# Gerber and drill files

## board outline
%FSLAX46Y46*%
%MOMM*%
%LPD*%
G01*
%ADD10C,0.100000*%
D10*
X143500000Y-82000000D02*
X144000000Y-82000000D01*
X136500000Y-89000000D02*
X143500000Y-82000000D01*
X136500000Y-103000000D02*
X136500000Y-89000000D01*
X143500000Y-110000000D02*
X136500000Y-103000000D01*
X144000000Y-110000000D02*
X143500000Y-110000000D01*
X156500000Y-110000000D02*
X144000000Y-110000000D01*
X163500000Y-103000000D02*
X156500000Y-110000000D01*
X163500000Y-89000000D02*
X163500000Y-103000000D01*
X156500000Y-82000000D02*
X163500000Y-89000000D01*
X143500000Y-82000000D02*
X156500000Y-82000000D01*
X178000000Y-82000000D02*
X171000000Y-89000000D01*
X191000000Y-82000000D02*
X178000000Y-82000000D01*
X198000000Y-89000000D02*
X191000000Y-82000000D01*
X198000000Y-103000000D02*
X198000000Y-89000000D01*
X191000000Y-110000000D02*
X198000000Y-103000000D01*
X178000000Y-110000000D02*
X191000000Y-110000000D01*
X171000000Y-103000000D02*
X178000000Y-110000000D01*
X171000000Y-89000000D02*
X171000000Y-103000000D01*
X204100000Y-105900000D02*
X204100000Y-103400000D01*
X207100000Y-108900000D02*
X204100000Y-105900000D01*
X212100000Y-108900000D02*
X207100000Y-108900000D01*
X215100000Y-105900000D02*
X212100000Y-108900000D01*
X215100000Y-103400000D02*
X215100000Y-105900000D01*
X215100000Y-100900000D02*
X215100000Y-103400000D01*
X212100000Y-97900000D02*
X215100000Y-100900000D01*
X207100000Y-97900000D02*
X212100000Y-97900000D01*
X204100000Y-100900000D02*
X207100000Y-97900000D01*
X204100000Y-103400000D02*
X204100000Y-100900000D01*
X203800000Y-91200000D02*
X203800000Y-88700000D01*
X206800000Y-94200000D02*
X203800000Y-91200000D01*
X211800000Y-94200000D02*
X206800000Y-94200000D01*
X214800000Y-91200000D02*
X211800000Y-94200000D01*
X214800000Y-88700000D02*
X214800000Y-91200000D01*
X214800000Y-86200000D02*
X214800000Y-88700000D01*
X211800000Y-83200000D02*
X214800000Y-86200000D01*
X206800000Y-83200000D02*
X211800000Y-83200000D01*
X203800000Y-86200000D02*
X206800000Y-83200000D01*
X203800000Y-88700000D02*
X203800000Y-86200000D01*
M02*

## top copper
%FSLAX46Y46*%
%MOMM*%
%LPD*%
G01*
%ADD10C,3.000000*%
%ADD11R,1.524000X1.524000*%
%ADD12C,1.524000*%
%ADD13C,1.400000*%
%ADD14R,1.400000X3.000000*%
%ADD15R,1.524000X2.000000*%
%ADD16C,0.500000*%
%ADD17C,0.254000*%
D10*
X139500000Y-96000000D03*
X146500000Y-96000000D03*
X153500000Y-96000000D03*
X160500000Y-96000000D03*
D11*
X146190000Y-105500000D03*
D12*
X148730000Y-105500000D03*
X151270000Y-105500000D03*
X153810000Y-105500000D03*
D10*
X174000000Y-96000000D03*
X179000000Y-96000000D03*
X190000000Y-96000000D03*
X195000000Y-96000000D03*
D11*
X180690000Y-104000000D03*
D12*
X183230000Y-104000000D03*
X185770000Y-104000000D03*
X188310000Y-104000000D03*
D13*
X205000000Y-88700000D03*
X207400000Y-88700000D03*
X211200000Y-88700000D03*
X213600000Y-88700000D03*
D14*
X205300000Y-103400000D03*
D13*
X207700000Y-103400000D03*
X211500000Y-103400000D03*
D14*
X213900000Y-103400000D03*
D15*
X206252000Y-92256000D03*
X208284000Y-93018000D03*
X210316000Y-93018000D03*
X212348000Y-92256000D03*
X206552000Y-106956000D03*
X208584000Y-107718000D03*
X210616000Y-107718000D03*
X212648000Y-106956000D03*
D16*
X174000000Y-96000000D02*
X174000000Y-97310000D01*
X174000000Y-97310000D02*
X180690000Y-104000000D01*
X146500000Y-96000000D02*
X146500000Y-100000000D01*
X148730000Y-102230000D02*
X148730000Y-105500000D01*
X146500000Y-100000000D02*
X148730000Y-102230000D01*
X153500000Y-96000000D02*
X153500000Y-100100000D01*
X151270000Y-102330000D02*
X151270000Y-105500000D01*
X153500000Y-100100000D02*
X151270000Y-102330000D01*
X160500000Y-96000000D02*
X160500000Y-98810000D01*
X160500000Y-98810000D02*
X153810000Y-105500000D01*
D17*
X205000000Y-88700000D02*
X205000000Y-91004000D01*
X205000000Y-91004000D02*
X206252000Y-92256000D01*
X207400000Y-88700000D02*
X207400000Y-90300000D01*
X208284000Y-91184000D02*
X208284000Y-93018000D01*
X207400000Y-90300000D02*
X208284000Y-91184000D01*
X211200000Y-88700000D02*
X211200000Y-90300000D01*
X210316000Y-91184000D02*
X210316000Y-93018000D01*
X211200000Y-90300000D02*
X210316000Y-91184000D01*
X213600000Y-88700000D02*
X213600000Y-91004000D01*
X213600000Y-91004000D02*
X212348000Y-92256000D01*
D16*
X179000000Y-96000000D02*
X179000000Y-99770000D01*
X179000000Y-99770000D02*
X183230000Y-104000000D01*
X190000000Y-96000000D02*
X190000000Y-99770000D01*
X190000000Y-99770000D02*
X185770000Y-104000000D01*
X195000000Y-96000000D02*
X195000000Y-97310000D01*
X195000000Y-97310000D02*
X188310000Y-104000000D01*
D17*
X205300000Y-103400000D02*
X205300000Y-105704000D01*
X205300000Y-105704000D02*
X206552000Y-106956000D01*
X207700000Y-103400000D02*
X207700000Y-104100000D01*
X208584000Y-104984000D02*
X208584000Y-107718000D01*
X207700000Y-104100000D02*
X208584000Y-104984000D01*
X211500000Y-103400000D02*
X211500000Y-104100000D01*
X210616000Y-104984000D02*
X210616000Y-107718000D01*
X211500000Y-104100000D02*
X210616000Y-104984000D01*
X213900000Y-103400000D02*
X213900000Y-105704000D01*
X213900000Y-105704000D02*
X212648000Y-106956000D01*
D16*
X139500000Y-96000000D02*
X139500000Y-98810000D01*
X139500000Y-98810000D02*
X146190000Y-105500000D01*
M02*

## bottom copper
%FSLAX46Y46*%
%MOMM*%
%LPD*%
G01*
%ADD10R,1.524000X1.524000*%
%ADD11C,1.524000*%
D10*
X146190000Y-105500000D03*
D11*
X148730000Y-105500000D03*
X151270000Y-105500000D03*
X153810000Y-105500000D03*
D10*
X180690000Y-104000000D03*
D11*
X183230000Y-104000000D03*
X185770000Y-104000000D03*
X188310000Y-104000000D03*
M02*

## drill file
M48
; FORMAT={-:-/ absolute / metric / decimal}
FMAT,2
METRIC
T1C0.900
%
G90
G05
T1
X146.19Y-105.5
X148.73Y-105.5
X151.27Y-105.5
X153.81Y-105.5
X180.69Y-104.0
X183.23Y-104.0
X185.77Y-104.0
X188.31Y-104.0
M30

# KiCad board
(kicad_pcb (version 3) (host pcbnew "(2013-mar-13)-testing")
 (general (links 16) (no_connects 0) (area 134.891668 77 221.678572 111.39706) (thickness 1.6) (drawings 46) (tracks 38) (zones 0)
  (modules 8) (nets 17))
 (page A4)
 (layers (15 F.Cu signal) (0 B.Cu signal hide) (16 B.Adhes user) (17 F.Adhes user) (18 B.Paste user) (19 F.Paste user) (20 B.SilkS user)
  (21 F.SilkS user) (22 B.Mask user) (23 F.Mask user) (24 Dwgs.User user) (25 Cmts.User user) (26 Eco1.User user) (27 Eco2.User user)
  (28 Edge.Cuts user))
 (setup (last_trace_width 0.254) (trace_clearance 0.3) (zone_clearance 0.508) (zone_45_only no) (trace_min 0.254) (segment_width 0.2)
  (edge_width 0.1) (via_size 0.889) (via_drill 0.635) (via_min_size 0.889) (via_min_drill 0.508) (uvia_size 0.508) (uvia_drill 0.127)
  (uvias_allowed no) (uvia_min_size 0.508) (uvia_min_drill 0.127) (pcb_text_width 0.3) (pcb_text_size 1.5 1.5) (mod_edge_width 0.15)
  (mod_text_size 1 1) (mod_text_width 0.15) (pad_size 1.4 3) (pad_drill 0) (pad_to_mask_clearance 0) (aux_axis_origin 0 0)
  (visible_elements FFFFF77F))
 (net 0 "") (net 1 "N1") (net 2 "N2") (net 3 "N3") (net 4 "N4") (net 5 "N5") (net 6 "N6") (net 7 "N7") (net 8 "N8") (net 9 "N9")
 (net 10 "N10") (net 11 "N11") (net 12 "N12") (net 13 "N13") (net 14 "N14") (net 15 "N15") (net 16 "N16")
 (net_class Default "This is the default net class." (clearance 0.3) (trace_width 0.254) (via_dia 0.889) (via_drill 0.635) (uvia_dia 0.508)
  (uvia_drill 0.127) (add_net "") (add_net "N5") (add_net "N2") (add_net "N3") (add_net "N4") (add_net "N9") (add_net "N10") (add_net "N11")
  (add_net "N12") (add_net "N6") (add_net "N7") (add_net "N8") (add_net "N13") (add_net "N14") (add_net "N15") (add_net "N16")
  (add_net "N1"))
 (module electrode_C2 (layer F.Cu) (at 150 96)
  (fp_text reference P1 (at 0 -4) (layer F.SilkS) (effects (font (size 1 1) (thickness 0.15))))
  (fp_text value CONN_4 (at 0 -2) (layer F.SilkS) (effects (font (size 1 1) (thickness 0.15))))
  (pad 1 smd circle (at -10.5 0) (size 3 3) (layers F.Cu F.Paste F.Mask) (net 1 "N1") (solder_mask_margin 0.1))
  (pad 2 smd circle (at -3.5 0) (size 3 3) (layers F.Cu F.Paste F.Mask) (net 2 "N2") (solder_mask_margin 0.1))
  (pad 3 smd circle (at 3.5 0) (size 3 3) (layers F.Cu F.Paste F.Mask) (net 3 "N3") (solder_mask_margin 0.1))
  (pad 4 smd circle (at 10.5 0) (size 3 3) (layers F.Cu F.Paste F.Mask) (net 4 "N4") (solder_mask_margin 0.1)))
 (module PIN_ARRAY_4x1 (layer F.Cu) (at 150 105.5)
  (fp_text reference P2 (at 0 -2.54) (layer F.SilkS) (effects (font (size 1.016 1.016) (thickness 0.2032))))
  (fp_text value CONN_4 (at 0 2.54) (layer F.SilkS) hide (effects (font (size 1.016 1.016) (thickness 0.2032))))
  (pad 1 thru_hole rect (at -3.81 0) (size 1.524 1.524) (drill 0.9) (layers *.Cu *.Mask F.SilkS) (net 1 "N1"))
  (pad 2 thru_hole circle (at -1.27 0) (size 1.524 1.524) (drill 0.9) (layers *.Cu *.Mask F.SilkS) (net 2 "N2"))
  (pad 3 thru_hole circle (at 1.27 0) (size 1.524 1.524) (drill 0.9) (layers *.Cu *.Mask F.SilkS) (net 3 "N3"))
  (pad 4 thru_hole circle (at 3.81 0) (size 1.524 1.524) (drill 0.9) (layers *.Cu *.Mask F.SilkS) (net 4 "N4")))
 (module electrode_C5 (layer F.Cu) (at 184.5 96)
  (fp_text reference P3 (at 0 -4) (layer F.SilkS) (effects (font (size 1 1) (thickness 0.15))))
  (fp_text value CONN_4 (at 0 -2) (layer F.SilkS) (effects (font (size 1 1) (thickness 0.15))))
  (pad 1 smd circle (at -10.5 0) (size 3 3) (layers F.Cu F.Paste F.Mask) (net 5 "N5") (solder_mask_margin 0.1))
  (pad 2 smd circle (at -5.5 0) (size 3 3) (layers F.Cu F.Paste F.Mask) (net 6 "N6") (solder_mask_margin 0.1))
  (pad 3 smd circle (at 5.5 0) (size 3 3) (layers F.Cu F.Paste F.Mask) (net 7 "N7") (solder_mask_margin 0.1))
  (pad 4 smd circle (at 10.5 0) (size 3 3) (layers F.Cu F.Paste F.Mask) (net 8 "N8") (solder_mask_margin 0.1)))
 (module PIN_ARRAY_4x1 (layer F.Cu) (at 184.5 104)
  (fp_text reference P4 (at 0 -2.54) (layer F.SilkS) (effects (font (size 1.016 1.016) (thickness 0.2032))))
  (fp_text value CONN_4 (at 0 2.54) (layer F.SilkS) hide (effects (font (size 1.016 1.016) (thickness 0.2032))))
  (pad 1 thru_hole rect (at -3.81 0) (size 1.524 1.524) (drill 0.9) (layers *.Cu *.Mask F.SilkS) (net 5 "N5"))
  (pad 2 thru_hole circle (at -1.27 0) (size 1.524 1.524) (drill 0.9) (layers *.Cu *.Mask F.SilkS) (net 6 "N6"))
  (pad 3 thru_hole circle (at 1.27 0) (size 1.524 1.524) (drill 0.9) (layers *.Cu *.Mask F.SilkS) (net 7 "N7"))
  (pad 4 thru_hole circle (at 3.81 0) (size 1.524 1.524) (drill 0.9) (layers *.Cu *.Mask F.SilkS) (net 8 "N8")))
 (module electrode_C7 (layer F.Cu) (at 209.3 88.7)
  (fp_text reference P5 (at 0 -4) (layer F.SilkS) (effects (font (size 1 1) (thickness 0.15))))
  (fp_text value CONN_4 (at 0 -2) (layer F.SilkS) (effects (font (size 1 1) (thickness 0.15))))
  (pad 1 smd circle (at -4.3 0) (size 1.4 1.4) (layers F.Cu F.Paste F.Mask) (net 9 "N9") (solder_mask_margin 0.1))
  (pad 2 smd circle (at -1.9 0) (size 1.4 1.4) (layers F.Cu F.Paste F.Mask) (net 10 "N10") (solder_mask_margin 0.1))
  (pad 3 smd circle (at 1.9 0) (size 1.4 1.4) (layers F.Cu F.Paste F.Mask) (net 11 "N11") (solder_mask_margin 0.1))
  (pad 4 smd circle (at 4.3 0) (size 1.4 1.4) (layers F.Cu F.Paste F.Mask) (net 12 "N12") (solder_mask_margin 0.1)))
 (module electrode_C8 (layer F.Cu) (at 209.6 103.4)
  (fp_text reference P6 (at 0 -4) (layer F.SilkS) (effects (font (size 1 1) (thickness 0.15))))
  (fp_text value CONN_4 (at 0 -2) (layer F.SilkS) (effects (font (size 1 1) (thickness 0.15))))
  (pad 1 smd rect (at -4.3 0) (size 1.4 3) (layers F.Cu F.Paste F.Mask) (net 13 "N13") (solder_mask_margin 0.1))
  (pad 2 smd circle (at -1.9 0) (size 1.4 1.4) (layers F.Cu F.Paste F.Mask) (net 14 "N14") (solder_mask_margin 0.1))
  (pad 3 smd circle (at 1.9 0) (size 1.4 1.4) (layers F.Cu F.Paste F.Mask) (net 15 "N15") (solder_mask_margin 0.1))
  (pad 4 smd rect (at 4.3 0) (size 1.4 3) (layers F.Cu F.Paste F.Mask) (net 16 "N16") (solder_mask_margin 0.1)))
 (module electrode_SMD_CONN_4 (layer F.Cu) (at 209.3 88.7)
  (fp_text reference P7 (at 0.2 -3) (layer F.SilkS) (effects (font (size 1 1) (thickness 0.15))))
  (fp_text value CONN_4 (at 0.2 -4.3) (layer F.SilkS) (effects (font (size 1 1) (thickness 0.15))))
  (pad 1 smd rect (at -3.048 3.556) (size 1.524 2) (layers F.Cu F.Paste F.Mask) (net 9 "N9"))
  (pad 2 smd rect (at -1.016 4.318) (size 1.524 2) (layers F.Cu F.Paste F.Mask) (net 10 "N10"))
  (pad 3 smd rect (at 1.016 4.318) (size 1.524 2) (layers F.Cu F.Paste F.Mask) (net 11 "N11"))
  (pad 4 smd rect (at 3.048 3.556) (size 1.524 2) (layers F.Cu F.Paste F.Mask) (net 12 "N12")))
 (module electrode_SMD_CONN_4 (layer F.Cu) (at 209.6 103.4)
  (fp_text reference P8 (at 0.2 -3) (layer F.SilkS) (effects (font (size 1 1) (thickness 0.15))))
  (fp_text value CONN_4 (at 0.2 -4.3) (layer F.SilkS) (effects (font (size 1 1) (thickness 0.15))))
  (pad 1 smd rect (at -3.048 3.556) (size 1.524 2) (layers F.Cu F.Paste F.Mask) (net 13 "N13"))
  (pad 2 smd rect (at -1.016 4.318) (size 1.524 2) (layers F.Cu F.Paste F.Mask) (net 14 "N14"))
  (pad 3 smd rect (at 1.016 4.318) (size 1.524 2) (layers F.Cu F.Paste F.Mask) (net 15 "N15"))
  (pad 4 smd rect (at 3.048 3.556) (size 1.524 2) (layers F.Cu F.Paste F.Mask) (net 16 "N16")))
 (gr_line (start 143.5 82) (end 144 82) (angle 90) (layer Edge.Cuts) (width 0.1))
 (gr_line (start 136.5 89) (end 143.5 82) (angle 90) (layer Edge.Cuts) (width 0.1))
 (gr_line (start 136.5 103) (end 136.5 89) (angle 90) (layer Edge.Cuts) (width 0.1))
 (gr_line (start 143.5 110) (end 136.5 103) (angle 90) (layer Edge.Cuts) (width 0.1))
 (gr_line (start 144 110) (end 143.5 110) (angle 90) (layer Edge.Cuts) (width 0.1))
 (gr_line (start 156.5 110) (end 144 110) (angle 90) (layer Edge.Cuts) (width 0.1))
 (gr_line (start 163.5 103) (end 156.5 110) (angle 90) (layer Edge.Cuts) (width 0.1))
 (gr_line (start 163.5 89) (end 163.5 103) (angle 90) (layer Edge.Cuts) (width 0.1))
 (gr_line (start 156.5 82) (end 163.5 89) (angle 90) (layer Edge.Cuts) (width 0.1))
 (gr_line (start 143.5 82) (end 156.5 82) (angle 90) (layer Edge.Cuts) (width 0.1))
 (gr_line (start 178 82) (end 171 89) (angle 90) (layer Edge.Cuts) (width 0.1))
 (gr_line (start 191 82) (end 178 82) (angle 90) (layer Edge.Cuts) (width 0.1))
 (gr_line (start 198 89) (end 191 82) (angle 90) (layer Edge.Cuts) (width 0.1))
 (gr_line (start 198 103) (end 198 89) (angle 90) (layer Edge.Cuts) (width 0.1))
 (gr_line (start 191 110) (end 198 103) (angle 90) (layer Edge.Cuts) (width 0.1))
 (gr_line (start 178 110) (end 191 110) (angle 90) (layer Edge.Cuts) (width 0.1))
 (gr_line (start 171 103) (end 178 110) (angle 90) (layer Edge.Cuts) (width 0.1))
 (gr_line (start 171 89) (end 171 103) (angle 90) (layer Edge.Cuts) (width 0.1))
 (gr_line (start 204.1 105.9) (end 204.1 103.4) (angle 90) (layer Edge.Cuts) (width 0.1))
 (gr_line (start 207.1 108.9) (end 204.1 105.9) (angle 90) (layer Edge.Cuts) (width 0.1))
 (gr_line (start 212.1 108.9) (end 207.1 108.9) (angle 90) (layer Edge.Cuts) (width 0.1))
 (gr_line (start 215.1 105.9) (end 212.1 108.9) (angle 90) (layer Edge.Cuts) (width 0.1))
 (gr_line (start 215.1 103.4) (end 215.1 105.9) (angle 90) (layer Edge.Cuts) (width 0.1))
 (gr_line (start 215.1 100.9) (end 215.1 103.4) (angle 90) (layer Edge.Cuts) (width 0.1))
 (gr_line (start 212.1 97.9) (end 215.1 100.9) (angle 90) (layer Edge.Cuts) (width 0.1))
 (gr_line (start 207.1 97.9) (end 212.1 97.9) (angle 90) (layer Edge.Cuts) (width 0.1))
 (gr_line (start 204.1 100.9) (end 207.1 97.9) (angle 90) (layer Edge.Cuts) (width 0.1))
 (gr_line (start 204.1 103.4) (end 204.1 100.9) (angle 90) (layer Edge.Cuts) (width 0.1))
 (gr_line (start 203.8 91.2) (end 203.8 88.7) (angle 90) (layer Edge.Cuts) (width 0.1))
 (gr_line (start 206.8 94.2) (end 203.8 91.2) (angle 90) (layer Edge.Cuts) (width 0.1))
 (gr_line (start 211.8 94.2) (end 206.8 94.2) (angle 90) (layer Edge.Cuts) (width 0.1))
 (gr_line (start 214.8 91.2) (end 211.8 94.2) (angle 90) (layer Edge.Cuts) (width 0.1))
 (gr_line (start 214.8 88.7) (end 214.8 91.2) (angle 90) (layer Edge.Cuts) (width 0.1))
 (gr_line (start 214.8 86.2) (end 214.8 88.7) (angle 90) (layer Edge.Cuts) (width 0.1))
 (gr_line (start 211.8 83.2) (end 214.8 86.2) (angle 90) (layer Edge.Cuts) (width 0.1))
 (gr_line (start 206.8 83.2) (end 211.8 83.2) (angle 90) (layer Edge.Cuts) (width 0.1))
 (gr_line (start 203.8 86.2) (end 206.8 83.2) (angle 90) (layer Edge.Cuts) (width 0.1))
 (gr_line (start 203.8 88.7) (end 203.8 86.2) (angle 90) (layer Edge.Cuts) (width 0.1))
 (segment (start 174 96) (end 174 97.31) (width 0.5) (layer F.Cu) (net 5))
 (segment (start 174 97.31) (end 180.69 104) (width 0.5) (layer F.Cu) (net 5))
 (segment (start 146.5 96) (end 146.5 100) (width 0.5) (layer F.Cu) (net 2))
 (segment (start 148.73 102.23) (end 148.73 105.5) (width 0.5) (layer F.Cu) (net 2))
 (segment (start 146.5 100) (end 148.73 102.23) (width 0.5) (layer F.Cu) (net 2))
 (segment (start 153.5 96) (end 153.5 100.1) (width 0.5) (layer F.Cu) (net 3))
 (segment (start 151.27 102.33) (end 151.27 105.5) (width 0.5) (layer F.Cu) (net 3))
 (segment (start 153.5 100.1) (end 151.27 102.33) (width 0.5) (layer F.Cu) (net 3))
 (segment (start 160.5 96) (end 160.5 98.81) (width 0.5) (layer F.Cu) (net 4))
 (segment (start 160.5 98.81) (end 153.81 105.5) (width 0.5) (layer F.Cu) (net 4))
 (segment (start 205 88.7) (end 205 91.004) (width 0.254) (layer F.Cu) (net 9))
 (segment (start 205 91.004) (end 206.252 92.256) (width 0.254) (layer F.Cu) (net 9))
 (segment (start 207.4 88.7) (end 207.4 90.3) (width 0.254) (layer F.Cu) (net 10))
 (segment (start 208.284 91.184) (end 208.284 93.018) (width 0.254) (layer F.Cu) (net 10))
 (segment (start 207.4 90.3) (end 208.284 91.184) (width 0.254) (layer F.Cu) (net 10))
 (segment (start 211.2 88.7) (end 211.2 90.3) (width 0.254) (layer F.Cu) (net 11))
 (segment (start 210.316 91.184) (end 210.316 93.018) (width 0.254) (layer F.Cu) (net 11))
 (segment (start 211.2 90.3) (end 210.316 91.184) (width 0.254) (layer F.Cu) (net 11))
 (segment (start 213.6 88.7) (end 213.6 91.004) (width 0.254) (layer F.Cu) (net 12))
 (segment (start 213.6 91.004) (end 212.348 92.256) (width 0.254) (layer F.Cu) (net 12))
 (segment (start 179 96) (end 179 99.77) (width 0.5) (layer F.Cu) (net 6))
 (segment (start 179 99.77) (end 183.23 104) (width 0.5) (layer F.Cu) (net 6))
 (segment (start 190 96) (end 190 99.77) (width 0.5) (layer F.Cu) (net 7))
 (segment (start 190 99.77) (end 185.77 104) (width 0.5) (layer F.Cu) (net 7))
 (segment (start 195 96) (end 195 97.31) (width 0.5) (layer F.Cu) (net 8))
 (segment (start 195 97.31) (end 188.31 104) (width 0.5) (layer F.Cu) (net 8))
 (segment (start 205.3 103.4) (end 205.3 105.704) (width 0.254) (layer F.Cu) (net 13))
 (segment (start 205.3 105.704) (end 206.552 106.956) (width 0.254) (layer F.Cu) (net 13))
 (segment (start 207.7 103.4) (end 207.7 104.1) (width 0.254) (layer F.Cu) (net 14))
 (segment (start 208.584 104.984) (end 208.584 107.718) (width 0.254) (layer F.Cu) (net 14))
 (segment (start 207.7 104.1) (end 208.584 104.984) (width 0.254) (layer F.Cu) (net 14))
 (segment (start 211.5 103.4) (end 211.5 104.1) (width 0.254) (layer F.Cu) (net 15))
 (segment (start 210.616 104.984) (end 210.616 107.718) (width 0.254) (layer F.Cu) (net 15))
 (segment (start 211.5 104.1) (end 210.616 104.984) (width 0.254) (layer F.Cu) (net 15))
 (segment (start 213.9 103.4) (end 213.9 105.704) (width 0.254) (layer F.Cu) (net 16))
 (segment (start 213.9 105.704) (end 212.648 106.956) (width 0.254) (layer F.Cu) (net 16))
 (segment (start 139.5 96) (end 139.5 98.81) (width 0.5) (layer F.Cu) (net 1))
 (segment (start 139.5 98.81) (end 146.19 105.5) (width 0.5) (layer F.Cu) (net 1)))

